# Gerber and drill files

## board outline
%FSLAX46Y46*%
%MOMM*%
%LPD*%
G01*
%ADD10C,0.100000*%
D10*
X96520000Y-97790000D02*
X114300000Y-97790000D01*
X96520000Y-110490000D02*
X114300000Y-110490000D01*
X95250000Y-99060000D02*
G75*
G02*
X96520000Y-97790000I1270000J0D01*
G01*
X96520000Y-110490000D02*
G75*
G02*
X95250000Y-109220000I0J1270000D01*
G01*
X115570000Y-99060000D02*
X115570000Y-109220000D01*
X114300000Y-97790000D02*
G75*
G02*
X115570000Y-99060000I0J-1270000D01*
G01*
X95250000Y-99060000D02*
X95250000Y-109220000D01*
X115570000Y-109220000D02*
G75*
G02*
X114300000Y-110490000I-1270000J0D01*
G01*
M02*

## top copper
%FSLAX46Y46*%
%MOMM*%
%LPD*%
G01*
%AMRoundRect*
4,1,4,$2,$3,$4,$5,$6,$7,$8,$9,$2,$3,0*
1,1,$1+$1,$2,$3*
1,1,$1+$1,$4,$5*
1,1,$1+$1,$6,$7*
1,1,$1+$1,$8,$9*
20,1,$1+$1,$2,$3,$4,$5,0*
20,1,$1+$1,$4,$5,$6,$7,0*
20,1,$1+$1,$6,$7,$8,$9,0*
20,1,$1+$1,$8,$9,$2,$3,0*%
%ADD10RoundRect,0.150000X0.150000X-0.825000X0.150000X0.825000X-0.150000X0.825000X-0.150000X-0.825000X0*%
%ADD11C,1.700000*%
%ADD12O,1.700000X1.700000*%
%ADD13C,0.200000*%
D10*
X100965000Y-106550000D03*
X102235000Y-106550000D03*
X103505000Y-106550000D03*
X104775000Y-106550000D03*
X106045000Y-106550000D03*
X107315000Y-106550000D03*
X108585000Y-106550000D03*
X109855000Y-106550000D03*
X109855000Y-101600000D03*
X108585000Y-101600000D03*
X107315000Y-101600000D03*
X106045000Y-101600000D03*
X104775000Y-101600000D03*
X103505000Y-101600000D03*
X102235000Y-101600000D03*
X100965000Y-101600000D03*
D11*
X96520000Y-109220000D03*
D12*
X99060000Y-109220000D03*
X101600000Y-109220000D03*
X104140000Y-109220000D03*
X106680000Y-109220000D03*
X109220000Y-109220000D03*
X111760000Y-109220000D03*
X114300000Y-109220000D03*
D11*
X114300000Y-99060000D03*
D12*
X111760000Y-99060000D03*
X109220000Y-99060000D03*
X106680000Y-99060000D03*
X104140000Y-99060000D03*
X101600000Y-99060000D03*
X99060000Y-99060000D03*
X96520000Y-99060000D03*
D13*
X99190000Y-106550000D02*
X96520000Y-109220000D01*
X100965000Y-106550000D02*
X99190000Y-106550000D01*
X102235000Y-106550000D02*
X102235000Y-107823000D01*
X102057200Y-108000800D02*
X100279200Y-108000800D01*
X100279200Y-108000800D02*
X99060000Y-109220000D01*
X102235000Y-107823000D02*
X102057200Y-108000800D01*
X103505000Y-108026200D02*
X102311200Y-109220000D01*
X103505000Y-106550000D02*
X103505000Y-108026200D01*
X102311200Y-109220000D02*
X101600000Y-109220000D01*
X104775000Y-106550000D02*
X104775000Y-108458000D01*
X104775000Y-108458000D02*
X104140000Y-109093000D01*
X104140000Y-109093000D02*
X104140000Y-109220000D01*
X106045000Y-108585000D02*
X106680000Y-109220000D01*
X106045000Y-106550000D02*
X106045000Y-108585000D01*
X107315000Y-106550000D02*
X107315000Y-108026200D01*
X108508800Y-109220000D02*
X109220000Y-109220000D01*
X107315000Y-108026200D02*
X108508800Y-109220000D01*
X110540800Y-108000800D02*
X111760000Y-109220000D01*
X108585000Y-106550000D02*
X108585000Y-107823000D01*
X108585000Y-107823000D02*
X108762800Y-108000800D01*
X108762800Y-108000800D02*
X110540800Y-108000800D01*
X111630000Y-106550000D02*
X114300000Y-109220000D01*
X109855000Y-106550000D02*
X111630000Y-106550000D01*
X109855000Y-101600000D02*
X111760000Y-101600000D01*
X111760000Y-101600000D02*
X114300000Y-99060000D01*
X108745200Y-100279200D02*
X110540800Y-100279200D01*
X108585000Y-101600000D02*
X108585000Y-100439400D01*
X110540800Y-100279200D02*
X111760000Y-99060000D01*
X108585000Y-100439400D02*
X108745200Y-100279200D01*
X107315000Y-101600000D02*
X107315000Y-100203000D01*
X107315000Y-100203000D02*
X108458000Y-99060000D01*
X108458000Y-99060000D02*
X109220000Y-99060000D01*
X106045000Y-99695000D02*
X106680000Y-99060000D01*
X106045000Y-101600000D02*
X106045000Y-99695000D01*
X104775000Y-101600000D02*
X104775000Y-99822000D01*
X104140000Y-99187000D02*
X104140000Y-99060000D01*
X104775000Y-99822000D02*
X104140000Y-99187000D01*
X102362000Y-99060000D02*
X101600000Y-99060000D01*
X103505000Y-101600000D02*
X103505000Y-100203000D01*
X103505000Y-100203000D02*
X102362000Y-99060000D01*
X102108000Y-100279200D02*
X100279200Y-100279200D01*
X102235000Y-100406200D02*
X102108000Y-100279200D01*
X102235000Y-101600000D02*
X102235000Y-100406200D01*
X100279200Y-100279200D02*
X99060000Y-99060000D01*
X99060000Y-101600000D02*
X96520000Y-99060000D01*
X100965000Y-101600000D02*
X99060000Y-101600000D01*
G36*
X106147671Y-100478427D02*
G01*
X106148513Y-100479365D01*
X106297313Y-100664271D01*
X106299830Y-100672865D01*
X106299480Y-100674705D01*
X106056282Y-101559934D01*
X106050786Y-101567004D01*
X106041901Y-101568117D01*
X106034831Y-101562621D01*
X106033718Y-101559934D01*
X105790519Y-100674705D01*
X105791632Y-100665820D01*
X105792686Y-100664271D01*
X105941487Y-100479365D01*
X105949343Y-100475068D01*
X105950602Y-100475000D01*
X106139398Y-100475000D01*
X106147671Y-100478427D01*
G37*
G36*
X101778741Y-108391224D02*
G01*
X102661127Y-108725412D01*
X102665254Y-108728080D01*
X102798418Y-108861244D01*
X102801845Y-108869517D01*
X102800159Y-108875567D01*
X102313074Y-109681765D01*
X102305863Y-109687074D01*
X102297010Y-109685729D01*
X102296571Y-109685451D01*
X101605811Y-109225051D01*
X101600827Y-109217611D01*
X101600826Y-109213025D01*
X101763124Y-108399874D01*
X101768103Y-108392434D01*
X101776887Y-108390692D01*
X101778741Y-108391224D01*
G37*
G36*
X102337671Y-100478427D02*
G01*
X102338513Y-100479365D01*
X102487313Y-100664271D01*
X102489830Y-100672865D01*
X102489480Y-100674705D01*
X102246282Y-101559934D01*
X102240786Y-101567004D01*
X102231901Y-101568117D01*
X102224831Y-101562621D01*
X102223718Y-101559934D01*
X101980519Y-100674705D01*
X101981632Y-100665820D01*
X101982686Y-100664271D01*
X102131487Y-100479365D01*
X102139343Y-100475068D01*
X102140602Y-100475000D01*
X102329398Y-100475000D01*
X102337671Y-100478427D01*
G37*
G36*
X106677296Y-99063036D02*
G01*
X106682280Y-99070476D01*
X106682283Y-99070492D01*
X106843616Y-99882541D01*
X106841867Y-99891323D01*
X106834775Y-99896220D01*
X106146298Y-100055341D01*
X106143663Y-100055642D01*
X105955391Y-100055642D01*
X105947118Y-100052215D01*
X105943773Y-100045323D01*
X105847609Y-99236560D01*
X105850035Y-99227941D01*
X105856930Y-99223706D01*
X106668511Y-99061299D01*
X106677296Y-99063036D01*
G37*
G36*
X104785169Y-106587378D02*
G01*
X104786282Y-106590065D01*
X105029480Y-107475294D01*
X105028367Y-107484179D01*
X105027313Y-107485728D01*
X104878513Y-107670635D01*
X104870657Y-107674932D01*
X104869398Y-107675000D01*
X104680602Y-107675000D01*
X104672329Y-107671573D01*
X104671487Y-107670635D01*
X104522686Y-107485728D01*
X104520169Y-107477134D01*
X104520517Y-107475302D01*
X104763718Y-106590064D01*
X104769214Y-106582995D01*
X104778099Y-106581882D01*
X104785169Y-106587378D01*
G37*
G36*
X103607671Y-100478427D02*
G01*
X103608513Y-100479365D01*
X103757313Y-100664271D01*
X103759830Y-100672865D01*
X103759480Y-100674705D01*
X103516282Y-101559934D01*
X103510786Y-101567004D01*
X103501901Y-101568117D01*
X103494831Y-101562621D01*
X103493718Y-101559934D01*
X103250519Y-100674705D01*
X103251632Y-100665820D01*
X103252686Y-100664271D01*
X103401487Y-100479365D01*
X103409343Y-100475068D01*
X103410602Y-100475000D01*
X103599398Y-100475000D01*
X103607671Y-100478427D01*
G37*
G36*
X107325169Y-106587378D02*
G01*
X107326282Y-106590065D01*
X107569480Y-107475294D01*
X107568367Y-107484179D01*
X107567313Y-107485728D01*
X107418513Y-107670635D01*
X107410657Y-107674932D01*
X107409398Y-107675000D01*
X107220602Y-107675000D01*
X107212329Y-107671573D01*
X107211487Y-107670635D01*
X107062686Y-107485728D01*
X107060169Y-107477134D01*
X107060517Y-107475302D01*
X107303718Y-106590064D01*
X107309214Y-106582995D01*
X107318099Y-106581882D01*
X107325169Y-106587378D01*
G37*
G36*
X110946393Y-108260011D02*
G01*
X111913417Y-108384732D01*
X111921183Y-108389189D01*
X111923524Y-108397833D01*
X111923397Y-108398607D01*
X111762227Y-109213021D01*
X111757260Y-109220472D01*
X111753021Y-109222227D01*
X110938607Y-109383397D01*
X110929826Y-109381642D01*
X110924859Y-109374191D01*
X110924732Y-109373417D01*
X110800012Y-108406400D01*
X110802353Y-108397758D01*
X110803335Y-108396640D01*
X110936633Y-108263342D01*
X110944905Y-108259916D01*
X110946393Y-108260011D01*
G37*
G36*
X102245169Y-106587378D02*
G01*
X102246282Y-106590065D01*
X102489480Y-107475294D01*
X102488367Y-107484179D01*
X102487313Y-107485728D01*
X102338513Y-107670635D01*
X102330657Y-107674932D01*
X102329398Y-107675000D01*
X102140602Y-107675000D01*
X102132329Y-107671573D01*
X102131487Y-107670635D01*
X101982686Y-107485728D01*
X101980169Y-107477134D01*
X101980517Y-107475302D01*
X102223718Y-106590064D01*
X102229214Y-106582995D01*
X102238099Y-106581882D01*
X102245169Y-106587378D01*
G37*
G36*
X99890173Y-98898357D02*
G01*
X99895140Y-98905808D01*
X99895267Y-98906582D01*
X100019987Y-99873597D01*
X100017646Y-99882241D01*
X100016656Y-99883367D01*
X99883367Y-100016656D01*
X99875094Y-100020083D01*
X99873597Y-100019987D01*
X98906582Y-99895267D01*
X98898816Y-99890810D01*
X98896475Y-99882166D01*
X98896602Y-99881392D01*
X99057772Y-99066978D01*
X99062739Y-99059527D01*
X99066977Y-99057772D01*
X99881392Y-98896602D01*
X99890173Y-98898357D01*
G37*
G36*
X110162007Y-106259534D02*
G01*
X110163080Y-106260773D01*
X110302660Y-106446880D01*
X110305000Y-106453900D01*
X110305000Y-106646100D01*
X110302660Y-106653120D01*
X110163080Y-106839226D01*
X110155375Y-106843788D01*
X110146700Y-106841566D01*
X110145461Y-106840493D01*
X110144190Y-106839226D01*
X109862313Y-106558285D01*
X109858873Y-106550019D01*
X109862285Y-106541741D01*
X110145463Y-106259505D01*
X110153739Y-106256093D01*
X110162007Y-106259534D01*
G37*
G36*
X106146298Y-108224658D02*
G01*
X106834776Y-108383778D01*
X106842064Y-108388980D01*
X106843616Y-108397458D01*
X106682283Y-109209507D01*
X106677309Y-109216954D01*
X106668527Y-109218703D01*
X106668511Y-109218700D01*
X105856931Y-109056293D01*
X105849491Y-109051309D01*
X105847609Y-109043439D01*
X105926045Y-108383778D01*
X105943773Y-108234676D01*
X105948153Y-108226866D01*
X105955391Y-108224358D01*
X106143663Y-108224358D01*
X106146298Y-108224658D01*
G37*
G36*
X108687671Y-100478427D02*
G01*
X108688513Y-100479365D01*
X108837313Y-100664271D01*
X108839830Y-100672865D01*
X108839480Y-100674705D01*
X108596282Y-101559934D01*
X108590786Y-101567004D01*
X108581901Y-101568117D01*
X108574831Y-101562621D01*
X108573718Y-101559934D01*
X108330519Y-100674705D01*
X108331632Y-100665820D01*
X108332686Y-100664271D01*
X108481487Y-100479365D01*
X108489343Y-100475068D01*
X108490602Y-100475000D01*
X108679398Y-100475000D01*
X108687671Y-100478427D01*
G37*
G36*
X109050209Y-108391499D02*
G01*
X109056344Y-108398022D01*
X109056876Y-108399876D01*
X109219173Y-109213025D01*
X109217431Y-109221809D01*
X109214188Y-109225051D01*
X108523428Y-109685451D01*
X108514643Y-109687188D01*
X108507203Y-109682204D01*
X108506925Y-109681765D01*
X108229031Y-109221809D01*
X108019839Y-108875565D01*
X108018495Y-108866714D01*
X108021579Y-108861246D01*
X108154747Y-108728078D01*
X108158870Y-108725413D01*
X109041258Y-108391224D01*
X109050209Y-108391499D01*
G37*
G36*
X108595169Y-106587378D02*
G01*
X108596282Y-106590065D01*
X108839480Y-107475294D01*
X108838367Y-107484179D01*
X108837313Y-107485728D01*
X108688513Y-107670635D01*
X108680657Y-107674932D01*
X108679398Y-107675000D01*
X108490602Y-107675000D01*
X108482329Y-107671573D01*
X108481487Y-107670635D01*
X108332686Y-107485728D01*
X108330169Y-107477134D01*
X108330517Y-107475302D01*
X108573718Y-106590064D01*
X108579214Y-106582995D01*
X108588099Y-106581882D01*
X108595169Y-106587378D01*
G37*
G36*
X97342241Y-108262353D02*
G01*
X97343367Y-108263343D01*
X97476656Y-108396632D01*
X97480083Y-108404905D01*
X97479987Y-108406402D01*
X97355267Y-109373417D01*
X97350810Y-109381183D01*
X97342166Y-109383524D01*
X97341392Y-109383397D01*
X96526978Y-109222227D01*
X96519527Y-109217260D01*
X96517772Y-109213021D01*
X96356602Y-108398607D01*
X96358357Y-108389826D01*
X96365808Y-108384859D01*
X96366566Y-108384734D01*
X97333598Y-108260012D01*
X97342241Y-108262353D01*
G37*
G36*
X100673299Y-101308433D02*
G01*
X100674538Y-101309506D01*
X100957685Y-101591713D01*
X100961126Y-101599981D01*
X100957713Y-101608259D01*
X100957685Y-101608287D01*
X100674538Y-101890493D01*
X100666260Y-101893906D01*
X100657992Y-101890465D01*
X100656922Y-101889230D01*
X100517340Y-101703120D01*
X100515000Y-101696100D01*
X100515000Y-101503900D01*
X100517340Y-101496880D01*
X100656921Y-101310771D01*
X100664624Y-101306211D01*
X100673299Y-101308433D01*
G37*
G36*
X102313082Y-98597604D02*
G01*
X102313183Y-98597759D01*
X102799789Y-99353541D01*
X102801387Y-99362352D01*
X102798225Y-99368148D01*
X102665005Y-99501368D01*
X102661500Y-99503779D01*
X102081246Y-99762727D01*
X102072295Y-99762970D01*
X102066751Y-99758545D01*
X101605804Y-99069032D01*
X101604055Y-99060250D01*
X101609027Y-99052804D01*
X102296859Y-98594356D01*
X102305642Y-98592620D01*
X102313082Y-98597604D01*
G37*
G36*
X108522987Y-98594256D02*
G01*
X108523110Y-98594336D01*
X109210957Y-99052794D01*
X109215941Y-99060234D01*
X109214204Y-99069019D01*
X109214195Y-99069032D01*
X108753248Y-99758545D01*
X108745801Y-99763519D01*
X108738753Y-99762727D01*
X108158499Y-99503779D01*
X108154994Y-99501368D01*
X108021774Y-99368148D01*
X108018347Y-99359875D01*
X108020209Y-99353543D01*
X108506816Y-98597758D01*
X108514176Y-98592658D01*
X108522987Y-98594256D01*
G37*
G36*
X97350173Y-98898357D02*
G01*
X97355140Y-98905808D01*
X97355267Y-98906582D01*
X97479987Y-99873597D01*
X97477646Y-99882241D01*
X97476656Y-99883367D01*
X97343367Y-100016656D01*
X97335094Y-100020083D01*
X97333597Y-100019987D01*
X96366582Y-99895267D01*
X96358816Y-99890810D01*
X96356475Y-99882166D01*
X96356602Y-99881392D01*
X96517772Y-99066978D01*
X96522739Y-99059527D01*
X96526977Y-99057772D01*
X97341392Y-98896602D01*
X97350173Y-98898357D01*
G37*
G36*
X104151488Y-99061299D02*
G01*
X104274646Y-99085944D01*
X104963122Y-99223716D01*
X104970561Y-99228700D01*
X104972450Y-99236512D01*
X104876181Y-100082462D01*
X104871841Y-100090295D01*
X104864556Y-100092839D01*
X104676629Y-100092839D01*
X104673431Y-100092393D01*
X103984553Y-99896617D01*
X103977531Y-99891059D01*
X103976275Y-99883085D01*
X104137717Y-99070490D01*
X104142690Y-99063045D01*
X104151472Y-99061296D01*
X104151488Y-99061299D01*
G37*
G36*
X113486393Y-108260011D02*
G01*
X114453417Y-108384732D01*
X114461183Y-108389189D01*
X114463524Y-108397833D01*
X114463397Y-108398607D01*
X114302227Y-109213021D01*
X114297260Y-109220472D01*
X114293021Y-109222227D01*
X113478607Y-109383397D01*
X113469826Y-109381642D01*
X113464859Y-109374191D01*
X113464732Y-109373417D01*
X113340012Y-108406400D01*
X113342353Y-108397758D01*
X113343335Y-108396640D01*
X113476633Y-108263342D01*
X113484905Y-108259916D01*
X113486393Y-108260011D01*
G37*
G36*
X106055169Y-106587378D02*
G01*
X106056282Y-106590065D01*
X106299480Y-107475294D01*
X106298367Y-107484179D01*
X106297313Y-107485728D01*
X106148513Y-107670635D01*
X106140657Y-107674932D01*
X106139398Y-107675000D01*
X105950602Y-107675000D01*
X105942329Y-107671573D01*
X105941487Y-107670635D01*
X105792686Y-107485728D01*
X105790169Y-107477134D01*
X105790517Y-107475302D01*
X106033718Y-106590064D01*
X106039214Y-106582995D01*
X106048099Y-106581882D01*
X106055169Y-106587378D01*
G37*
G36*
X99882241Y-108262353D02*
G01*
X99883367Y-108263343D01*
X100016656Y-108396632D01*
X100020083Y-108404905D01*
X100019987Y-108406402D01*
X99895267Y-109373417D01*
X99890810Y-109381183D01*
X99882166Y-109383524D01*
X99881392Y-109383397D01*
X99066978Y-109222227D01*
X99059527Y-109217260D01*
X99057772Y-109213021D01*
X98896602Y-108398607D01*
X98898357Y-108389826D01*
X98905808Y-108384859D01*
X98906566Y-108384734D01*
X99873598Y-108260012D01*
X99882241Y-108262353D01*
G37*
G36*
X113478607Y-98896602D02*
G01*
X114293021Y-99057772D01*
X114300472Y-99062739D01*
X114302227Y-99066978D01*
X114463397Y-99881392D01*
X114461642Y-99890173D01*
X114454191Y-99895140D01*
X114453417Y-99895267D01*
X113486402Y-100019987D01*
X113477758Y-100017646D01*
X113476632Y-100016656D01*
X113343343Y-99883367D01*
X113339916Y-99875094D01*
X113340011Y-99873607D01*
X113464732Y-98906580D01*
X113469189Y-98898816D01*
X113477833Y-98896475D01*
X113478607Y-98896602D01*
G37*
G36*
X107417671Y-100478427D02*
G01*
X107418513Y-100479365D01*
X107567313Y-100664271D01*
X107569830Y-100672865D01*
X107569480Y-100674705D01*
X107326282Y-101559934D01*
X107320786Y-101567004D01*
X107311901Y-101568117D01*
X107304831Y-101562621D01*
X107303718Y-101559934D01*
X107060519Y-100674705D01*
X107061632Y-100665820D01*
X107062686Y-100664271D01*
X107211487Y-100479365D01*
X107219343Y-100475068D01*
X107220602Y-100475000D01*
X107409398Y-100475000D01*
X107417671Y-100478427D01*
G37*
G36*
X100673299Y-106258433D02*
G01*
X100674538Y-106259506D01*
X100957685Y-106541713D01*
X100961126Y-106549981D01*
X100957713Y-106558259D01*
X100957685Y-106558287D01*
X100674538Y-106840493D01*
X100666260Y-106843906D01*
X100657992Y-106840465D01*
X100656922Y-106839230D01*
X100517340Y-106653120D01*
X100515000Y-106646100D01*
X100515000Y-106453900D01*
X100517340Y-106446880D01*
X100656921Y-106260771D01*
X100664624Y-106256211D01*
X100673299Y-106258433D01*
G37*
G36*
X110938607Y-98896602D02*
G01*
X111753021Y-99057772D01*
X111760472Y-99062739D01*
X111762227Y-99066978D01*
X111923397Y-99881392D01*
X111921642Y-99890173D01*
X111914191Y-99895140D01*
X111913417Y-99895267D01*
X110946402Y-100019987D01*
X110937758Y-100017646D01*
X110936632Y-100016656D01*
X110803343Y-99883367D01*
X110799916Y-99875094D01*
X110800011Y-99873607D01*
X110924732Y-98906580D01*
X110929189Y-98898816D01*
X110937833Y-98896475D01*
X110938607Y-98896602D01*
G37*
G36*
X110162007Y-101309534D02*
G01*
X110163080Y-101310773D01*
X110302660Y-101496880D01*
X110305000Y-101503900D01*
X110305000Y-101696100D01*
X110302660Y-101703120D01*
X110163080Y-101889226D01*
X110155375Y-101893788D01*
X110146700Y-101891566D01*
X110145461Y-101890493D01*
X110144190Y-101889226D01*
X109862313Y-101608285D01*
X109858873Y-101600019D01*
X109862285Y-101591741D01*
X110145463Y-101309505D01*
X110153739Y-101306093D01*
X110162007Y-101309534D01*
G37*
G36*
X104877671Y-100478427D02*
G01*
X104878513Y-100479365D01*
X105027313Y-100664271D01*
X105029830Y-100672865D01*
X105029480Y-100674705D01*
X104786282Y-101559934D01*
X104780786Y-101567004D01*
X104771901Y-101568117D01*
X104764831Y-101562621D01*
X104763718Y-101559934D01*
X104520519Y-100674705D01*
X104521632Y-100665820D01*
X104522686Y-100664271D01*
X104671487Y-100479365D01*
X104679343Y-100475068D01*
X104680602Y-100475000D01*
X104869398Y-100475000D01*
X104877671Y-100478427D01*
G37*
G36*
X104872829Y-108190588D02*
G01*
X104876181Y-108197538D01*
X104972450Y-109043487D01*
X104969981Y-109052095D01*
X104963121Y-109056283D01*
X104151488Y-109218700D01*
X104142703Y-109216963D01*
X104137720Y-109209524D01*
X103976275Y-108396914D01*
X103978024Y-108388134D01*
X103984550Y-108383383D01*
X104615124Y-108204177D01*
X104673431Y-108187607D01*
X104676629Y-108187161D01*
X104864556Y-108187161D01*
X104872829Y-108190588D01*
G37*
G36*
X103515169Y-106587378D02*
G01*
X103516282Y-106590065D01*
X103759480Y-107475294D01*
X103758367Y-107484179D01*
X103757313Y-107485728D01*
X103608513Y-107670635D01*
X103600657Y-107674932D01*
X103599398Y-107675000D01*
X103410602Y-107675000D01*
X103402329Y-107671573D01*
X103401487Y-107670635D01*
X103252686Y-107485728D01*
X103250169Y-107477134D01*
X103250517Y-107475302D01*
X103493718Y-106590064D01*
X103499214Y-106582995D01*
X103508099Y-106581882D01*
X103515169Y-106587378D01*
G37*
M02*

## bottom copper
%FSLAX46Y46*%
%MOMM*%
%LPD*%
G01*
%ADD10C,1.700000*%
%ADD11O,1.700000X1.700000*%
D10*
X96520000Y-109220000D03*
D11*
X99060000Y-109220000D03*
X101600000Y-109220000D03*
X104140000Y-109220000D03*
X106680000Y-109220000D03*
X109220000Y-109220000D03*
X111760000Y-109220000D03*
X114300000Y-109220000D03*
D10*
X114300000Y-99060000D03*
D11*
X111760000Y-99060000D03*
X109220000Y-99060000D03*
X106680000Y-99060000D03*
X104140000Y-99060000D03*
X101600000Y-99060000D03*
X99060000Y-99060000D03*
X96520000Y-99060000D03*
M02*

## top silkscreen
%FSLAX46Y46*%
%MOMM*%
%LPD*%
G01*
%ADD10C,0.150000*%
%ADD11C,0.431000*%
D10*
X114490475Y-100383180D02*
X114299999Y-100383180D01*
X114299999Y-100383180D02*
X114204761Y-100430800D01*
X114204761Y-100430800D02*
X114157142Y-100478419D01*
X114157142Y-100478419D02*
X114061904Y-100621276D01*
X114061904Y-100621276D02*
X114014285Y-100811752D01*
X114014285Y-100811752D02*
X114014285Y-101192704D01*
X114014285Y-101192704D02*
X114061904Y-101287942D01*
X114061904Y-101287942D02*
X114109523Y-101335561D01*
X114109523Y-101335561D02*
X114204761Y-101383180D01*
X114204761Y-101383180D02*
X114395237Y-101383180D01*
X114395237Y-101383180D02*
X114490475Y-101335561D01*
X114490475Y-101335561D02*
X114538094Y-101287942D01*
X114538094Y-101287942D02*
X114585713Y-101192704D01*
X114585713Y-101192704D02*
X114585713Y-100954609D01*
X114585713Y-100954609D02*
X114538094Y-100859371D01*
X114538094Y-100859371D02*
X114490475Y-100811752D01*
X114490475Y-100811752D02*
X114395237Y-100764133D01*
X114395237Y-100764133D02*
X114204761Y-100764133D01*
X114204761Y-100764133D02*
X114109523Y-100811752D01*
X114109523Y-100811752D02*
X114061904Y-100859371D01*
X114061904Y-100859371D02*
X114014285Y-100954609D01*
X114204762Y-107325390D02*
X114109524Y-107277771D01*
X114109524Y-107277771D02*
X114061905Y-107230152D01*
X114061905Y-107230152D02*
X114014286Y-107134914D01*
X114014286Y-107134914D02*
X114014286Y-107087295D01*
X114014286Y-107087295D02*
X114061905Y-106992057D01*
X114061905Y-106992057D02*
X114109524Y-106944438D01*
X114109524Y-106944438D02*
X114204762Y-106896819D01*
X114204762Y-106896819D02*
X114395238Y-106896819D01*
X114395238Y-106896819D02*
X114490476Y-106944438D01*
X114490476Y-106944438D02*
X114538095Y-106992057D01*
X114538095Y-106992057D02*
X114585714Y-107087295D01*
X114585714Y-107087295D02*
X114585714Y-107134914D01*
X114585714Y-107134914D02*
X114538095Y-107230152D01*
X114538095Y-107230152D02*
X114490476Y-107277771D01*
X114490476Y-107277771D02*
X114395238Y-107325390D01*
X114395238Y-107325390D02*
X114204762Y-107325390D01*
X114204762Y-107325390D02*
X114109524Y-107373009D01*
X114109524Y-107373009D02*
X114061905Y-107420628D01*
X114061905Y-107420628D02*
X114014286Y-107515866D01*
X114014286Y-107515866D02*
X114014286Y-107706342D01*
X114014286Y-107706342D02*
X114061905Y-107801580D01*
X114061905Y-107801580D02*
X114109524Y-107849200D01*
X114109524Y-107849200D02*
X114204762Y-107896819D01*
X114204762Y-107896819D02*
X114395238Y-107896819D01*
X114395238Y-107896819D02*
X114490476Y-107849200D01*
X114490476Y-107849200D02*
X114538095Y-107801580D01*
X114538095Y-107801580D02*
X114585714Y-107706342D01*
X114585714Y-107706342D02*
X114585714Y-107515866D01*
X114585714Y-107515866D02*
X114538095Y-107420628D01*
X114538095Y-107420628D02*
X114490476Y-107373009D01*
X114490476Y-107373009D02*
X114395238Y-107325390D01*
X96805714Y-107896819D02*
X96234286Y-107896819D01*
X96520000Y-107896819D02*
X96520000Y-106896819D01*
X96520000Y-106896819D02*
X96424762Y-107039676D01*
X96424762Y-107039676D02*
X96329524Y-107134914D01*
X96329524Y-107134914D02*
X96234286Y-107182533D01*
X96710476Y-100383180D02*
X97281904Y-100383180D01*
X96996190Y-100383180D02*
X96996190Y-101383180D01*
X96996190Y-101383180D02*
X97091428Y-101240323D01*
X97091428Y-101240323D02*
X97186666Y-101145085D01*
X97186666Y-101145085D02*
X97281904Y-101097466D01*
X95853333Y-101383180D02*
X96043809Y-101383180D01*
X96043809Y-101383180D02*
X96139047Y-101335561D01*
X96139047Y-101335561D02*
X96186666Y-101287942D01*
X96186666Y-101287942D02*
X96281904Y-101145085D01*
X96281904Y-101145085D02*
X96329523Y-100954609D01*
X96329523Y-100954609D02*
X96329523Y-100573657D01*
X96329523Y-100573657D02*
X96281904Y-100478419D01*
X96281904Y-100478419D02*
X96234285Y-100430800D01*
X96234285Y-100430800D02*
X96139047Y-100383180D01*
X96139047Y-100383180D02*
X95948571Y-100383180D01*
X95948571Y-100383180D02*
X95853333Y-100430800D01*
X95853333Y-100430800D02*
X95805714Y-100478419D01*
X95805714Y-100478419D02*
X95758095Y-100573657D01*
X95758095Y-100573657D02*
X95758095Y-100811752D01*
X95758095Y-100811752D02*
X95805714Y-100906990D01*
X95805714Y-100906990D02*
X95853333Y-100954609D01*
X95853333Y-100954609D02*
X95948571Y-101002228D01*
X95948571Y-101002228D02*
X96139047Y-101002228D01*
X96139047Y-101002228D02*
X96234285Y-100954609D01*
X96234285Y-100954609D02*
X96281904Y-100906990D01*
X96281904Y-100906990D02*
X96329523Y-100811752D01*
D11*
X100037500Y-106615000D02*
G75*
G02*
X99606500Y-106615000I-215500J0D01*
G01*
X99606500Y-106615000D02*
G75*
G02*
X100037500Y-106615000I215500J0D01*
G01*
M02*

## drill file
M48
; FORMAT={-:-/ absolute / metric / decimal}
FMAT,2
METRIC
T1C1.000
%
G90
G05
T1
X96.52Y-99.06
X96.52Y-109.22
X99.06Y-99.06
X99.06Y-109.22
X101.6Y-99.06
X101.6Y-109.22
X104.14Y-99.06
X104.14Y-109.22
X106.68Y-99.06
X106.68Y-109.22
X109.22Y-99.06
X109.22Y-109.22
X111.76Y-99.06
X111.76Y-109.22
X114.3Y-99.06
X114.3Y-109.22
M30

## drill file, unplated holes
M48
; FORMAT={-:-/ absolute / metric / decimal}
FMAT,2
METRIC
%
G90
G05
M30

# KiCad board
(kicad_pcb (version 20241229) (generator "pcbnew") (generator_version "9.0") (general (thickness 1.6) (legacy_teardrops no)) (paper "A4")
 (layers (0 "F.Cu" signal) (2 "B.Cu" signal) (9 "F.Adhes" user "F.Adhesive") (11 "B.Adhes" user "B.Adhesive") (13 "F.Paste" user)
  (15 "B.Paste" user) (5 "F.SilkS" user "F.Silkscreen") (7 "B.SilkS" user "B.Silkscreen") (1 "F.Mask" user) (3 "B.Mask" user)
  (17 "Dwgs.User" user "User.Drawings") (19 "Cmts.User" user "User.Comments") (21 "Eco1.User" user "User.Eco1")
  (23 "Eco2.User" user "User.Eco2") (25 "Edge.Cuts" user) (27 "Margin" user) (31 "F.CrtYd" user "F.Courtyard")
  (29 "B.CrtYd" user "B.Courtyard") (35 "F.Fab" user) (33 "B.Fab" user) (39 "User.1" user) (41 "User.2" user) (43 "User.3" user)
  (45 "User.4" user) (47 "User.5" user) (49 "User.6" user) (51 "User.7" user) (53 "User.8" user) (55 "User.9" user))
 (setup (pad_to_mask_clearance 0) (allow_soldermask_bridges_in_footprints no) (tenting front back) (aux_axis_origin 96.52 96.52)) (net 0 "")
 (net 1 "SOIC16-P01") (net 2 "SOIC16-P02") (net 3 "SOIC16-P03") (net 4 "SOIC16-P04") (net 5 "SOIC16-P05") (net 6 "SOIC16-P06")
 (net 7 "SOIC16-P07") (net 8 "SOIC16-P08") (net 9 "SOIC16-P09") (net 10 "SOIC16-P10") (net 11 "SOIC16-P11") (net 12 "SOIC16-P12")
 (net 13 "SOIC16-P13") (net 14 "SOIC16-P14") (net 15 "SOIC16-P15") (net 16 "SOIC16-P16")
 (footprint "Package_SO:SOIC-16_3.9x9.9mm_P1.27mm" (layer "F.Cu") (at 105.41 104.075 90)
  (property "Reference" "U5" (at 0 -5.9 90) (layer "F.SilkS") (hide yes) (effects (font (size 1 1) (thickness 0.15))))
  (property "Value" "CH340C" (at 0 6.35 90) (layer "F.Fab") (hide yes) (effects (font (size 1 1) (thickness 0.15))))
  (fp_circle (center -2.54 -5.588) (end -2.159 -5.588) (stroke (width 0.1) (type solid)) (fill yes) (layer "F.SilkS"))
  (pad "1" smd roundrect (at -2.475 -4.445 90) (size 1.95 0.6) (layers "F.Cu" "F.Mask" "F.Paste") (roundrect_rratio 0.25)
   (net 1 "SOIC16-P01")
   (teardrops (best_length_ratio 0.25) (max_length 1) (best_width_ratio 1) (max_width 2) (curved_edges no) (filter_ratio 0.9) (enabled yes)
    (allow_two_segments yes) (prefer_zone_connections yes)))
  (pad "2" smd roundrect (at -2.475 -3.175 90) (size 1.95 0.6) (layers "F.Cu" "F.Mask" "F.Paste") (roundrect_rratio 0.25)
   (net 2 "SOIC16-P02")
   (teardrops (best_length_ratio 0.25) (max_length 1) (best_width_ratio 1) (max_width 2) (curved_edges no) (filter_ratio 0.9) (enabled yes)
    (allow_two_segments yes) (prefer_zone_connections yes)))
  (pad "3" smd roundrect (at -2.475 -1.905 90) (size 1.95 0.6) (layers "F.Cu" "F.Mask" "F.Paste") (roundrect_rratio 0.25)
   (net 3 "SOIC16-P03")
   (teardrops (best_length_ratio 0.25) (max_length 1) (best_width_ratio 1) (max_width 2) (curved_edges no) (filter_ratio 0.9) (enabled yes)
    (allow_two_segments yes) (prefer_zone_connections yes)))
  (pad "4" smd roundrect (at -2.475 -0.635 90) (size 1.95 0.6) (layers "F.Cu" "F.Mask" "F.Paste") (roundrect_rratio 0.25)
   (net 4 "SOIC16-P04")
   (teardrops (best_length_ratio 0.25) (max_length 1) (best_width_ratio 1) (max_width 2) (curved_edges no) (filter_ratio 0.9) (enabled yes)
    (allow_two_segments yes) (prefer_zone_connections yes)))
  (pad "5" smd roundrect (at -2.475 0.635 90) (size 1.95 0.6) (layers "F.Cu" "F.Mask" "F.Paste") (roundrect_rratio 0.25)
   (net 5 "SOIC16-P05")
   (teardrops (best_length_ratio 0.25) (max_length 1) (best_width_ratio 1) (max_width 2) (curved_edges no) (filter_ratio 0.9) (enabled yes)
    (allow_two_segments yes) (prefer_zone_connections yes)))
  (pad "6" smd roundrect (at -2.475 1.905 90) (size 1.95 0.6) (layers "F.Cu" "F.Mask" "F.Paste") (roundrect_rratio 0.25)
   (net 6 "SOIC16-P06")
   (teardrops (best_length_ratio 0.25) (max_length 1) (best_width_ratio 1) (max_width 2) (curved_edges no) (filter_ratio 0.9) (enabled yes)
    (allow_two_segments yes) (prefer_zone_connections yes)))
  (pad "7" smd roundrect (at -2.475 3.175 90) (size 1.95 0.6) (layers "F.Cu" "F.Mask" "F.Paste") (roundrect_rratio 0.25)
   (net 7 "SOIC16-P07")
   (teardrops (best_length_ratio 0.25) (max_length 1) (best_width_ratio 1) (max_width 2) (curved_edges no) (filter_ratio 0.9) (enabled yes)
    (allow_two_segments yes) (prefer_zone_connections yes)))
  (pad "8" smd roundrect (at -2.475 4.445 90) (size 1.95 0.6) (layers "F.Cu" "F.Mask" "F.Paste") (roundrect_rratio 0.25)
   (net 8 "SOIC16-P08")
   (teardrops (best_length_ratio 0.25) (max_length 1) (best_width_ratio 1) (max_width 2) (curved_edges no) (filter_ratio 0.9) (enabled yes)
    (allow_two_segments yes) (prefer_zone_connections yes)))
  (pad "9" smd roundrect (at 2.475 4.445 90) (size 1.95 0.6) (layers "F.Cu" "F.Mask" "F.Paste") (roundrect_rratio 0.25) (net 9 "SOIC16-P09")
   (teardrops (best_length_ratio 0.25) (max_length 1) (best_width_ratio 1) (max_width 2) (curved_edges no) (filter_ratio 0.9) (enabled yes)
    (allow_two_segments yes) (prefer_zone_connections yes)))
  (pad "10" smd roundrect (at 2.475 3.175 90) (size 1.95 0.6) (layers "F.Cu" "F.Mask" "F.Paste") (roundrect_rratio 0.25)
   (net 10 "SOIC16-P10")
   (teardrops (best_length_ratio 0.25) (max_length 1) (best_width_ratio 1) (max_width 2) (curved_edges no) (filter_ratio 0.9) (enabled yes)
    (allow_two_segments yes) (prefer_zone_connections yes)))
  (pad "11" smd roundrect (at 2.475 1.905 90) (size 1.95 0.6) (layers "F.Cu" "F.Mask" "F.Paste") (roundrect_rratio 0.25)
   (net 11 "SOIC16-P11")
   (teardrops (best_length_ratio 0.25) (max_length 1) (best_width_ratio 1) (max_width 2) (curved_edges no) (filter_ratio 0.9) (enabled yes)
    (allow_two_segments yes) (prefer_zone_connections yes)))
  (pad "12" smd roundrect (at 2.475 0.635 90) (size 1.95 0.6) (layers "F.Cu" "F.Mask" "F.Paste") (roundrect_rratio 0.25)
   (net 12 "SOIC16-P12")
   (teardrops (best_length_ratio 0.25) (max_length 1) (best_width_ratio 1) (max_width 2) (curved_edges no) (filter_ratio 0.9) (enabled yes)
    (allow_two_segments yes) (prefer_zone_connections yes)))
  (pad "13" smd roundrect (at 2.475 -0.635 90) (size 1.95 0.6) (layers "F.Cu" "F.Mask" "F.Paste") (roundrect_rratio 0.25)
   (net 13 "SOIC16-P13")
   (teardrops (best_length_ratio 0.25) (max_length 1) (best_width_ratio 1) (max_width 2) (curved_edges no) (filter_ratio 0.9) (enabled yes)
    (allow_two_segments yes) (prefer_zone_connections yes)))
  (pad "14" smd roundrect (at 2.475 -1.905 90) (size 1.95 0.6) (layers "F.Cu" "F.Mask" "F.Paste") (roundrect_rratio 0.25)
   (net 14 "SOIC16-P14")
   (teardrops (best_length_ratio 0.25) (max_length 1) (best_width_ratio 1) (max_width 2) (curved_edges no) (filter_ratio 0.9) (enabled yes)
    (allow_two_segments yes) (prefer_zone_connections yes)))
  (pad "15" smd roundrect (at 2.475 -3.175 90) (size 1.95 0.6) (layers "F.Cu" "F.Mask" "F.Paste") (roundrect_rratio 0.25)
   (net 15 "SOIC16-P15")
   (teardrops (best_length_ratio 0.25) (max_length 1) (best_width_ratio 1) (max_width 2) (curved_edges no) (filter_ratio 0.9) (enabled yes)
    (allow_two_segments yes) (prefer_zone_connections yes)))
  (pad "16" smd roundrect (at 2.475 -4.445 90) (size 1.95 0.6) (layers "F.Cu" "F.Mask" "F.Paste") (roundrect_rratio 0.25)
   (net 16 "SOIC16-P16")
   (teardrops (best_length_ratio 0.25) (max_length 1) (best_width_ratio 1) (max_width 2) (curved_edges no) (filter_ratio 0.9) (enabled yes)
    (allow_two_segments yes) (prefer_zone_connections yes))))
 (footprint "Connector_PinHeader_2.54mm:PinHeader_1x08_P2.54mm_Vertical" (layer "B.Cu") (at 96.52 109.22 -90)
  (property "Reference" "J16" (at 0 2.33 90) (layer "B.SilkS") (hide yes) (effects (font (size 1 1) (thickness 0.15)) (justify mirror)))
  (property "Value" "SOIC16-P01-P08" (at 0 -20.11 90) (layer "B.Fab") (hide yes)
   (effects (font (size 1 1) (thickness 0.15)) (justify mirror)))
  (pad "1" thru_hole circle (at 0 0 270) (size 1.7 1.7) (drill 1) (layers "*.Cu" "*.Mask") (remove_unused_layers no) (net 1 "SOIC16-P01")
   (teardrops (best_length_ratio 0.25) (max_length 1) (best_width_ratio 1) (max_width 2) (curved_edges no) (filter_ratio 0.9) (enabled yes)
    (allow_two_segments yes) (prefer_zone_connections yes)))
  (pad "2" thru_hole oval (at 0 -2.54 270) (size 1.7 1.7) (drill 1) (layers "*.Cu" "*.Mask") (remove_unused_layers no) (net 2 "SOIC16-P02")
   (teardrops (best_length_ratio 0.25) (max_length 1) (best_width_ratio 1) (max_width 2) (curved_edges no) (filter_ratio 0.9) (enabled yes)
    (allow_two_segments yes) (prefer_zone_connections yes)))
  (pad "3" thru_hole oval (at 0 -5.08 270) (size 1.7 1.7) (drill 1) (layers "*.Cu" "*.Mask") (remove_unused_layers no) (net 3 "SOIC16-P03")
   (teardrops (best_length_ratio 0.25) (max_length 1) (best_width_ratio 1) (max_width 2) (curved_edges no) (filter_ratio 0.9) (enabled yes)
    (allow_two_segments yes) (prefer_zone_connections yes)))
  (pad "4" thru_hole oval (at 0 -7.62 270) (size 1.7 1.7) (drill 1) (layers "*.Cu" "*.Mask") (remove_unused_layers no) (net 4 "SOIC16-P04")
   (teardrops (best_length_ratio 0.25) (max_length 1) (best_width_ratio 1) (max_width 2) (curved_edges no) (filter_ratio 0.9) (enabled yes)
    (allow_two_segments yes) (prefer_zone_connections yes)))
  (pad "5" thru_hole oval (at 0 -10.16 270) (size 1.7 1.7) (drill 1) (layers "*.Cu" "*.Mask") (remove_unused_layers no) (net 5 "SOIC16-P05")
   (teardrops (best_length_ratio 0.25) (max_length 1) (best_width_ratio 1) (max_width 2) (curved_edges no) (filter_ratio 0.9) (enabled yes)
    (allow_two_segments yes) (prefer_zone_connections yes)))
  (pad "6" thru_hole oval (at 0 -12.7 270) (size 1.7 1.7) (drill 1) (layers "*.Cu" "*.Mask") (remove_unused_layers no) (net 6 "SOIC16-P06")
   (teardrops (best_length_ratio 0.25) (max_length 1) (best_width_ratio 1) (max_width 2) (curved_edges no) (filter_ratio 0.9) (enabled yes)
    (allow_two_segments yes) (prefer_zone_connections yes)))
  (pad "7" thru_hole oval (at 0 -15.24 270) (size 1.7 1.7) (drill 1) (layers "*.Cu" "*.Mask") (remove_unused_layers no) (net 7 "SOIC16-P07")
   (teardrops (best_length_ratio 0.25) (max_length 1) (best_width_ratio 1) (max_width 2) (curved_edges no) (filter_ratio 0.9) (enabled yes)
    (allow_two_segments yes) (prefer_zone_connections yes)))
  (pad "8" thru_hole oval (at 0 -17.78 270) (size 1.7 1.7) (drill 1) (layers "*.Cu" "*.Mask") (remove_unused_layers no) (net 8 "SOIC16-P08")
   (teardrops (best_length_ratio 0.25) (max_length 1) (best_width_ratio 1) (max_width 2) (curved_edges no) (filter_ratio 0.9) (enabled yes)
    (allow_two_segments yes) (prefer_zone_connections yes))))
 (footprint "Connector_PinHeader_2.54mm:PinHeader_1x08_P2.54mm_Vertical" (layer "B.Cu") (at 114.3 99.06 90)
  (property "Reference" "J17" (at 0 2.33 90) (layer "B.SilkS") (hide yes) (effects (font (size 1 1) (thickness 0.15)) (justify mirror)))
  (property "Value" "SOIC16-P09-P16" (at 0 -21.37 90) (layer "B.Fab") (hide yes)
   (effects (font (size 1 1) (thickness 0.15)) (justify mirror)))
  (pad "1" thru_hole circle (at 0 0 90) (size 1.7 1.7) (drill 1) (layers "*.Cu" "*.Mask") (remove_unused_layers no) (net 9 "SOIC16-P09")
   (teardrops (best_length_ratio 0.25) (max_length 1) (best_width_ratio 1) (max_width 2) (curved_edges no) (filter_ratio 0.9) (enabled yes)
    (allow_two_segments yes) (prefer_zone_connections yes)))
  (pad "2" thru_hole oval (at 0 -2.54 90) (size 1.7 1.7) (drill 1) (layers "*.Cu" "*.Mask") (remove_unused_layers no) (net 10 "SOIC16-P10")
   (teardrops (best_length_ratio 0.25) (max_length 1) (best_width_ratio 1) (max_width 2) (curved_edges no) (filter_ratio 0.9) (enabled yes)
    (allow_two_segments yes) (prefer_zone_connections yes)))
  (pad "3" thru_hole oval (at 0 -5.08 90) (size 1.7 1.7) (drill 1) (layers "*.Cu" "*.Mask") (remove_unused_layers no) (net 11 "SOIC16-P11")
   (teardrops (best_length_ratio 0.25) (max_length 1) (best_width_ratio 1) (max_width 2) (curved_edges no) (filter_ratio 0.9) (enabled yes)
    (allow_two_segments yes) (prefer_zone_connections yes)))
  (pad "4" thru_hole oval (at 0 -7.62 90) (size 1.7 1.7) (drill 1) (layers "*.Cu" "*.Mask") (remove_unused_layers no) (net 12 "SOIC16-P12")
   (teardrops (best_length_ratio 0.25) (max_length 1) (best_width_ratio 1) (max_width 2) (curved_edges no) (filter_ratio 0.9) (enabled yes)
    (allow_two_segments yes) (prefer_zone_connections yes)))
  (pad "5" thru_hole oval (at 0 -10.16 90) (size 1.7 1.7) (drill 1) (layers "*.Cu" "*.Mask") (remove_unused_layers no) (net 13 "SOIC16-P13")
   (teardrops (best_length_ratio 0.25) (max_length 1) (best_width_ratio 1) (max_width 2) (curved_edges no) (filter_ratio 0.9) (enabled yes)
    (allow_two_segments yes) (prefer_zone_connections yes)))
  (pad "6" thru_hole oval (at 0 -12.7 90) (size 1.7 1.7) (drill 1) (layers "*.Cu" "*.Mask") (remove_unused_layers no) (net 14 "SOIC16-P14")
   (teardrops (best_length_ratio 0.25) (max_length 1) (best_width_ratio 1) (max_width 2) (curved_edges no) (filter_ratio 0.9) (enabled yes)
    (allow_two_segments yes) (prefer_zone_connections yes)))
  (pad "7" thru_hole oval (at 0 -15.24 90) (size 1.7 1.7) (drill 1) (layers "*.Cu" "*.Mask") (remove_unused_layers no) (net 15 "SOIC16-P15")
   (teardrops (best_length_ratio 0.25) (max_length 1) (best_width_ratio 1) (max_width 2) (curved_edges no) (filter_ratio 0.9) (enabled yes)
    (allow_two_segments yes) (prefer_zone_connections yes)))
  (pad "8" thru_hole oval (at 0 -17.78 90) (size 1.7 1.7) (drill 1) (layers "*.Cu" "*.Mask") (remove_unused_layers no) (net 16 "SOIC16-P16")
   (teardrops (best_length_ratio 0.25) (max_length 1) (best_width_ratio 1) (max_width 2) (curved_edges no) (filter_ratio 0.9) (enabled yes)
    (allow_two_segments yes) (prefer_zone_connections yes))))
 (gr_line (start 96.52 97.79) (end 114.3 97.79) (stroke (width 0.1) (type solid)) (layer "Edge.Cuts"))
 (gr_line (start 96.52 110.49) (end 114.3 110.49) (stroke (width 0.1) (type solid)) (layer "Edge.Cuts"))
 (gr_arc (start 95.25 99.06) (mid 95.621974 98.161974) (end 96.52 97.79) (stroke (width 0.1) (type default)) (layer "Edge.Cuts"))
 (gr_arc (start 96.52 110.49) (mid 95.621974 110.118026) (end 95.25 109.22) (stroke (width 0.1) (type default)) (layer "Edge.Cuts"))
 (gr_line (start 115.57 99.06) (end 115.57 109.22) (stroke (width 0.1) (type solid)) (layer "Edge.Cuts"))
 (gr_arc (start 114.3 97.79) (mid 115.198026 98.161974) (end 115.57 99.06) (stroke (width 0.1) (type default)) (layer "Edge.Cuts"))
 (gr_line (start 95.25 99.06) (end 95.25 109.22) (stroke (width 0.1) (type solid)) (layer "Edge.Cuts"))
 (gr_arc (start 115.57 109.22) (mid 115.198026 110.118026) (end 114.3 110.49) (stroke (width 0.1) (type default)) (layer "Edge.Cuts"))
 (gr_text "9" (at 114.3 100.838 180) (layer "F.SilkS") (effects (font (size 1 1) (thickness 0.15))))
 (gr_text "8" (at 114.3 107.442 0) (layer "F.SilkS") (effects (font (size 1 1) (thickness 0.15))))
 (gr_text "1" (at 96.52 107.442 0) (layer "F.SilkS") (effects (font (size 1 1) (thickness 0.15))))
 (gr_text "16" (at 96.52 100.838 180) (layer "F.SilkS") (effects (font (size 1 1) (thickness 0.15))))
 (segment (start 99.19 106.55) (end 96.52 109.22) (width 0.2) (layer "F.Cu") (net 1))
 (segment (start 100.965 106.55) (end 99.19 106.55) (width 0.2) (layer "F.Cu") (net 1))
 (segment (start 102.235 106.55) (end 102.235 107.823) (width 0.2) (layer "F.Cu") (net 2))
 (segment (start 102.0572 108.0008) (end 100.2792 108.0008) (width 0.2) (layer "F.Cu") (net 2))
 (segment (start 100.2792 108.0008) (end 99.06 109.22) (width 0.2) (layer "F.Cu") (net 2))
 (segment (start 102.235 107.823) (end 102.0572 108.0008) (width 0.2) (layer "F.Cu") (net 2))
 (segment (start 103.505 108.0262) (end 102.3112 109.22) (width 0.2) (layer "F.Cu") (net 3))
 (segment (start 103.505 106.55) (end 103.505 108.0262) (width 0.2) (layer "F.Cu") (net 3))
 (segment (start 102.3112 109.22) (end 101.6 109.22) (width 0.2) (layer "F.Cu") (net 3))
 (segment (start 104.775 106.55) (end 104.775 108.458) (width 0.2) (layer "F.Cu") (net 4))
 (segment (start 104.775 108.458) (end 104.14 109.093) (width 0.2) (layer "F.Cu") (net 4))
 (segment (start 104.14 109.093) (end 104.14 109.22) (width 0.2) (layer "F.Cu") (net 4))
 (segment (start 106.045 108.585) (end 106.68 109.22) (width 0.2) (layer "F.Cu") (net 5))
 (segment (start 106.045 106.55) (end 106.045 108.585) (width 0.2) (layer "F.Cu") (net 5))
 (segment (start 107.315 106.55) (end 107.315 108.0262) (width 0.2) (layer "F.Cu") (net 6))
 (segment (start 108.5088 109.22) (end 109.22 109.22) (width 0.2) (layer "F.Cu") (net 6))
 (segment (start 107.315 108.0262) (end 108.5088 109.22) (width 0.2) (layer "F.Cu") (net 6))
 (segment (start 110.5408 108.0008) (end 111.76 109.22) (width 0.2) (layer "F.Cu") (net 7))
 (segment (start 108.585 106.55) (end 108.585 107.823) (width 0.2) (layer "F.Cu") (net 7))
 (segment (start 108.585 107.823) (end 108.7628 108.0008) (width 0.2) (layer "F.Cu") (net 7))
 (segment (start 108.7628 108.0008) (end 110.5408 108.0008) (width 0.2) (layer "F.Cu") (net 7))
 (segment (start 111.63 106.55) (end 114.3 109.22) (width 0.2) (layer "F.Cu") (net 8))
 (segment (start 109.855 106.55) (end 111.63 106.55) (width 0.2) (layer "F.Cu") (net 8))
 (segment (start 109.855 101.6) (end 111.76 101.6) (width 0.2) (layer "F.Cu") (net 9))
 (segment (start 111.76 101.6) (end 114.3 99.06) (width 0.2) (layer "F.Cu") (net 9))
 (segment (start 108.7452 100.2792) (end 110.5408 100.2792) (width 0.2) (layer "F.Cu") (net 10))
 (segment (start 108.585 101.6) (end 108.585 100.4394) (width 0.2) (layer "F.Cu") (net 10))
 (segment (start 110.5408 100.2792) (end 111.76 99.06) (width 0.2) (layer "F.Cu") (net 10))
 (segment (start 108.585 100.4394) (end 108.7452 100.2792) (width 0.2) (layer "F.Cu") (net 10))
 (segment (start 107.315 101.6) (end 107.315 100.203) (width 0.2) (layer "F.Cu") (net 11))
 (segment (start 107.315 100.203) (end 108.458 99.06) (width 0.2) (layer "F.Cu") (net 11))
 (segment (start 108.458 99.06) (end 109.22 99.06) (width 0.2) (layer "F.Cu") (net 11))
 (segment (start 106.045 99.695) (end 106.68 99.06) (width 0.2) (layer "F.Cu") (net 12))
 (segment (start 106.045 101.6) (end 106.045 99.695) (width 0.2) (layer "F.Cu") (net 12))
 (segment (start 104.775 101.6) (end 104.775 99.822) (width 0.2) (layer "F.Cu") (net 13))
 (segment (start 104.14 99.187) (end 104.14 99.06) (width 0.2) (layer "F.Cu") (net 13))
 (segment (start 104.775 99.822) (end 104.14 99.187) (width 0.2) (layer "F.Cu") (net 13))
 (segment (start 102.362 99.06) (end 101.6 99.06) (width 0.2) (layer "F.Cu") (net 14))
 (segment (start 103.505 101.6) (end 103.505 100.203) (width 0.2) (layer "F.Cu") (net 14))
 (segment (start 103.505 100.203) (end 102.362 99.06) (width 0.2) (layer "F.Cu") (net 14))
 (segment (start 102.108 100.2792) (end 100.2792 100.2792) (width 0.2) (layer "F.Cu") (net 15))
 (segment (start 102.235 100.4062) (end 102.108 100.2792) (width 0.2) (layer "F.Cu") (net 15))
 (segment (start 102.235 101.6) (end 102.235 100.4062) (width 0.2) (layer "F.Cu") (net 15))
 (segment (start 100.2792 100.2792) (end 99.06 99.06) (width 0.2) (layer "F.Cu") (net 15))
 (segment (start 99.06 101.6) (end 96.52 99.06) (width 0.2) (layer "F.Cu") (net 16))
 (segment (start 100.965 101.6) (end 99.06 101.6) (width 0.2) (layer "F.Cu") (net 16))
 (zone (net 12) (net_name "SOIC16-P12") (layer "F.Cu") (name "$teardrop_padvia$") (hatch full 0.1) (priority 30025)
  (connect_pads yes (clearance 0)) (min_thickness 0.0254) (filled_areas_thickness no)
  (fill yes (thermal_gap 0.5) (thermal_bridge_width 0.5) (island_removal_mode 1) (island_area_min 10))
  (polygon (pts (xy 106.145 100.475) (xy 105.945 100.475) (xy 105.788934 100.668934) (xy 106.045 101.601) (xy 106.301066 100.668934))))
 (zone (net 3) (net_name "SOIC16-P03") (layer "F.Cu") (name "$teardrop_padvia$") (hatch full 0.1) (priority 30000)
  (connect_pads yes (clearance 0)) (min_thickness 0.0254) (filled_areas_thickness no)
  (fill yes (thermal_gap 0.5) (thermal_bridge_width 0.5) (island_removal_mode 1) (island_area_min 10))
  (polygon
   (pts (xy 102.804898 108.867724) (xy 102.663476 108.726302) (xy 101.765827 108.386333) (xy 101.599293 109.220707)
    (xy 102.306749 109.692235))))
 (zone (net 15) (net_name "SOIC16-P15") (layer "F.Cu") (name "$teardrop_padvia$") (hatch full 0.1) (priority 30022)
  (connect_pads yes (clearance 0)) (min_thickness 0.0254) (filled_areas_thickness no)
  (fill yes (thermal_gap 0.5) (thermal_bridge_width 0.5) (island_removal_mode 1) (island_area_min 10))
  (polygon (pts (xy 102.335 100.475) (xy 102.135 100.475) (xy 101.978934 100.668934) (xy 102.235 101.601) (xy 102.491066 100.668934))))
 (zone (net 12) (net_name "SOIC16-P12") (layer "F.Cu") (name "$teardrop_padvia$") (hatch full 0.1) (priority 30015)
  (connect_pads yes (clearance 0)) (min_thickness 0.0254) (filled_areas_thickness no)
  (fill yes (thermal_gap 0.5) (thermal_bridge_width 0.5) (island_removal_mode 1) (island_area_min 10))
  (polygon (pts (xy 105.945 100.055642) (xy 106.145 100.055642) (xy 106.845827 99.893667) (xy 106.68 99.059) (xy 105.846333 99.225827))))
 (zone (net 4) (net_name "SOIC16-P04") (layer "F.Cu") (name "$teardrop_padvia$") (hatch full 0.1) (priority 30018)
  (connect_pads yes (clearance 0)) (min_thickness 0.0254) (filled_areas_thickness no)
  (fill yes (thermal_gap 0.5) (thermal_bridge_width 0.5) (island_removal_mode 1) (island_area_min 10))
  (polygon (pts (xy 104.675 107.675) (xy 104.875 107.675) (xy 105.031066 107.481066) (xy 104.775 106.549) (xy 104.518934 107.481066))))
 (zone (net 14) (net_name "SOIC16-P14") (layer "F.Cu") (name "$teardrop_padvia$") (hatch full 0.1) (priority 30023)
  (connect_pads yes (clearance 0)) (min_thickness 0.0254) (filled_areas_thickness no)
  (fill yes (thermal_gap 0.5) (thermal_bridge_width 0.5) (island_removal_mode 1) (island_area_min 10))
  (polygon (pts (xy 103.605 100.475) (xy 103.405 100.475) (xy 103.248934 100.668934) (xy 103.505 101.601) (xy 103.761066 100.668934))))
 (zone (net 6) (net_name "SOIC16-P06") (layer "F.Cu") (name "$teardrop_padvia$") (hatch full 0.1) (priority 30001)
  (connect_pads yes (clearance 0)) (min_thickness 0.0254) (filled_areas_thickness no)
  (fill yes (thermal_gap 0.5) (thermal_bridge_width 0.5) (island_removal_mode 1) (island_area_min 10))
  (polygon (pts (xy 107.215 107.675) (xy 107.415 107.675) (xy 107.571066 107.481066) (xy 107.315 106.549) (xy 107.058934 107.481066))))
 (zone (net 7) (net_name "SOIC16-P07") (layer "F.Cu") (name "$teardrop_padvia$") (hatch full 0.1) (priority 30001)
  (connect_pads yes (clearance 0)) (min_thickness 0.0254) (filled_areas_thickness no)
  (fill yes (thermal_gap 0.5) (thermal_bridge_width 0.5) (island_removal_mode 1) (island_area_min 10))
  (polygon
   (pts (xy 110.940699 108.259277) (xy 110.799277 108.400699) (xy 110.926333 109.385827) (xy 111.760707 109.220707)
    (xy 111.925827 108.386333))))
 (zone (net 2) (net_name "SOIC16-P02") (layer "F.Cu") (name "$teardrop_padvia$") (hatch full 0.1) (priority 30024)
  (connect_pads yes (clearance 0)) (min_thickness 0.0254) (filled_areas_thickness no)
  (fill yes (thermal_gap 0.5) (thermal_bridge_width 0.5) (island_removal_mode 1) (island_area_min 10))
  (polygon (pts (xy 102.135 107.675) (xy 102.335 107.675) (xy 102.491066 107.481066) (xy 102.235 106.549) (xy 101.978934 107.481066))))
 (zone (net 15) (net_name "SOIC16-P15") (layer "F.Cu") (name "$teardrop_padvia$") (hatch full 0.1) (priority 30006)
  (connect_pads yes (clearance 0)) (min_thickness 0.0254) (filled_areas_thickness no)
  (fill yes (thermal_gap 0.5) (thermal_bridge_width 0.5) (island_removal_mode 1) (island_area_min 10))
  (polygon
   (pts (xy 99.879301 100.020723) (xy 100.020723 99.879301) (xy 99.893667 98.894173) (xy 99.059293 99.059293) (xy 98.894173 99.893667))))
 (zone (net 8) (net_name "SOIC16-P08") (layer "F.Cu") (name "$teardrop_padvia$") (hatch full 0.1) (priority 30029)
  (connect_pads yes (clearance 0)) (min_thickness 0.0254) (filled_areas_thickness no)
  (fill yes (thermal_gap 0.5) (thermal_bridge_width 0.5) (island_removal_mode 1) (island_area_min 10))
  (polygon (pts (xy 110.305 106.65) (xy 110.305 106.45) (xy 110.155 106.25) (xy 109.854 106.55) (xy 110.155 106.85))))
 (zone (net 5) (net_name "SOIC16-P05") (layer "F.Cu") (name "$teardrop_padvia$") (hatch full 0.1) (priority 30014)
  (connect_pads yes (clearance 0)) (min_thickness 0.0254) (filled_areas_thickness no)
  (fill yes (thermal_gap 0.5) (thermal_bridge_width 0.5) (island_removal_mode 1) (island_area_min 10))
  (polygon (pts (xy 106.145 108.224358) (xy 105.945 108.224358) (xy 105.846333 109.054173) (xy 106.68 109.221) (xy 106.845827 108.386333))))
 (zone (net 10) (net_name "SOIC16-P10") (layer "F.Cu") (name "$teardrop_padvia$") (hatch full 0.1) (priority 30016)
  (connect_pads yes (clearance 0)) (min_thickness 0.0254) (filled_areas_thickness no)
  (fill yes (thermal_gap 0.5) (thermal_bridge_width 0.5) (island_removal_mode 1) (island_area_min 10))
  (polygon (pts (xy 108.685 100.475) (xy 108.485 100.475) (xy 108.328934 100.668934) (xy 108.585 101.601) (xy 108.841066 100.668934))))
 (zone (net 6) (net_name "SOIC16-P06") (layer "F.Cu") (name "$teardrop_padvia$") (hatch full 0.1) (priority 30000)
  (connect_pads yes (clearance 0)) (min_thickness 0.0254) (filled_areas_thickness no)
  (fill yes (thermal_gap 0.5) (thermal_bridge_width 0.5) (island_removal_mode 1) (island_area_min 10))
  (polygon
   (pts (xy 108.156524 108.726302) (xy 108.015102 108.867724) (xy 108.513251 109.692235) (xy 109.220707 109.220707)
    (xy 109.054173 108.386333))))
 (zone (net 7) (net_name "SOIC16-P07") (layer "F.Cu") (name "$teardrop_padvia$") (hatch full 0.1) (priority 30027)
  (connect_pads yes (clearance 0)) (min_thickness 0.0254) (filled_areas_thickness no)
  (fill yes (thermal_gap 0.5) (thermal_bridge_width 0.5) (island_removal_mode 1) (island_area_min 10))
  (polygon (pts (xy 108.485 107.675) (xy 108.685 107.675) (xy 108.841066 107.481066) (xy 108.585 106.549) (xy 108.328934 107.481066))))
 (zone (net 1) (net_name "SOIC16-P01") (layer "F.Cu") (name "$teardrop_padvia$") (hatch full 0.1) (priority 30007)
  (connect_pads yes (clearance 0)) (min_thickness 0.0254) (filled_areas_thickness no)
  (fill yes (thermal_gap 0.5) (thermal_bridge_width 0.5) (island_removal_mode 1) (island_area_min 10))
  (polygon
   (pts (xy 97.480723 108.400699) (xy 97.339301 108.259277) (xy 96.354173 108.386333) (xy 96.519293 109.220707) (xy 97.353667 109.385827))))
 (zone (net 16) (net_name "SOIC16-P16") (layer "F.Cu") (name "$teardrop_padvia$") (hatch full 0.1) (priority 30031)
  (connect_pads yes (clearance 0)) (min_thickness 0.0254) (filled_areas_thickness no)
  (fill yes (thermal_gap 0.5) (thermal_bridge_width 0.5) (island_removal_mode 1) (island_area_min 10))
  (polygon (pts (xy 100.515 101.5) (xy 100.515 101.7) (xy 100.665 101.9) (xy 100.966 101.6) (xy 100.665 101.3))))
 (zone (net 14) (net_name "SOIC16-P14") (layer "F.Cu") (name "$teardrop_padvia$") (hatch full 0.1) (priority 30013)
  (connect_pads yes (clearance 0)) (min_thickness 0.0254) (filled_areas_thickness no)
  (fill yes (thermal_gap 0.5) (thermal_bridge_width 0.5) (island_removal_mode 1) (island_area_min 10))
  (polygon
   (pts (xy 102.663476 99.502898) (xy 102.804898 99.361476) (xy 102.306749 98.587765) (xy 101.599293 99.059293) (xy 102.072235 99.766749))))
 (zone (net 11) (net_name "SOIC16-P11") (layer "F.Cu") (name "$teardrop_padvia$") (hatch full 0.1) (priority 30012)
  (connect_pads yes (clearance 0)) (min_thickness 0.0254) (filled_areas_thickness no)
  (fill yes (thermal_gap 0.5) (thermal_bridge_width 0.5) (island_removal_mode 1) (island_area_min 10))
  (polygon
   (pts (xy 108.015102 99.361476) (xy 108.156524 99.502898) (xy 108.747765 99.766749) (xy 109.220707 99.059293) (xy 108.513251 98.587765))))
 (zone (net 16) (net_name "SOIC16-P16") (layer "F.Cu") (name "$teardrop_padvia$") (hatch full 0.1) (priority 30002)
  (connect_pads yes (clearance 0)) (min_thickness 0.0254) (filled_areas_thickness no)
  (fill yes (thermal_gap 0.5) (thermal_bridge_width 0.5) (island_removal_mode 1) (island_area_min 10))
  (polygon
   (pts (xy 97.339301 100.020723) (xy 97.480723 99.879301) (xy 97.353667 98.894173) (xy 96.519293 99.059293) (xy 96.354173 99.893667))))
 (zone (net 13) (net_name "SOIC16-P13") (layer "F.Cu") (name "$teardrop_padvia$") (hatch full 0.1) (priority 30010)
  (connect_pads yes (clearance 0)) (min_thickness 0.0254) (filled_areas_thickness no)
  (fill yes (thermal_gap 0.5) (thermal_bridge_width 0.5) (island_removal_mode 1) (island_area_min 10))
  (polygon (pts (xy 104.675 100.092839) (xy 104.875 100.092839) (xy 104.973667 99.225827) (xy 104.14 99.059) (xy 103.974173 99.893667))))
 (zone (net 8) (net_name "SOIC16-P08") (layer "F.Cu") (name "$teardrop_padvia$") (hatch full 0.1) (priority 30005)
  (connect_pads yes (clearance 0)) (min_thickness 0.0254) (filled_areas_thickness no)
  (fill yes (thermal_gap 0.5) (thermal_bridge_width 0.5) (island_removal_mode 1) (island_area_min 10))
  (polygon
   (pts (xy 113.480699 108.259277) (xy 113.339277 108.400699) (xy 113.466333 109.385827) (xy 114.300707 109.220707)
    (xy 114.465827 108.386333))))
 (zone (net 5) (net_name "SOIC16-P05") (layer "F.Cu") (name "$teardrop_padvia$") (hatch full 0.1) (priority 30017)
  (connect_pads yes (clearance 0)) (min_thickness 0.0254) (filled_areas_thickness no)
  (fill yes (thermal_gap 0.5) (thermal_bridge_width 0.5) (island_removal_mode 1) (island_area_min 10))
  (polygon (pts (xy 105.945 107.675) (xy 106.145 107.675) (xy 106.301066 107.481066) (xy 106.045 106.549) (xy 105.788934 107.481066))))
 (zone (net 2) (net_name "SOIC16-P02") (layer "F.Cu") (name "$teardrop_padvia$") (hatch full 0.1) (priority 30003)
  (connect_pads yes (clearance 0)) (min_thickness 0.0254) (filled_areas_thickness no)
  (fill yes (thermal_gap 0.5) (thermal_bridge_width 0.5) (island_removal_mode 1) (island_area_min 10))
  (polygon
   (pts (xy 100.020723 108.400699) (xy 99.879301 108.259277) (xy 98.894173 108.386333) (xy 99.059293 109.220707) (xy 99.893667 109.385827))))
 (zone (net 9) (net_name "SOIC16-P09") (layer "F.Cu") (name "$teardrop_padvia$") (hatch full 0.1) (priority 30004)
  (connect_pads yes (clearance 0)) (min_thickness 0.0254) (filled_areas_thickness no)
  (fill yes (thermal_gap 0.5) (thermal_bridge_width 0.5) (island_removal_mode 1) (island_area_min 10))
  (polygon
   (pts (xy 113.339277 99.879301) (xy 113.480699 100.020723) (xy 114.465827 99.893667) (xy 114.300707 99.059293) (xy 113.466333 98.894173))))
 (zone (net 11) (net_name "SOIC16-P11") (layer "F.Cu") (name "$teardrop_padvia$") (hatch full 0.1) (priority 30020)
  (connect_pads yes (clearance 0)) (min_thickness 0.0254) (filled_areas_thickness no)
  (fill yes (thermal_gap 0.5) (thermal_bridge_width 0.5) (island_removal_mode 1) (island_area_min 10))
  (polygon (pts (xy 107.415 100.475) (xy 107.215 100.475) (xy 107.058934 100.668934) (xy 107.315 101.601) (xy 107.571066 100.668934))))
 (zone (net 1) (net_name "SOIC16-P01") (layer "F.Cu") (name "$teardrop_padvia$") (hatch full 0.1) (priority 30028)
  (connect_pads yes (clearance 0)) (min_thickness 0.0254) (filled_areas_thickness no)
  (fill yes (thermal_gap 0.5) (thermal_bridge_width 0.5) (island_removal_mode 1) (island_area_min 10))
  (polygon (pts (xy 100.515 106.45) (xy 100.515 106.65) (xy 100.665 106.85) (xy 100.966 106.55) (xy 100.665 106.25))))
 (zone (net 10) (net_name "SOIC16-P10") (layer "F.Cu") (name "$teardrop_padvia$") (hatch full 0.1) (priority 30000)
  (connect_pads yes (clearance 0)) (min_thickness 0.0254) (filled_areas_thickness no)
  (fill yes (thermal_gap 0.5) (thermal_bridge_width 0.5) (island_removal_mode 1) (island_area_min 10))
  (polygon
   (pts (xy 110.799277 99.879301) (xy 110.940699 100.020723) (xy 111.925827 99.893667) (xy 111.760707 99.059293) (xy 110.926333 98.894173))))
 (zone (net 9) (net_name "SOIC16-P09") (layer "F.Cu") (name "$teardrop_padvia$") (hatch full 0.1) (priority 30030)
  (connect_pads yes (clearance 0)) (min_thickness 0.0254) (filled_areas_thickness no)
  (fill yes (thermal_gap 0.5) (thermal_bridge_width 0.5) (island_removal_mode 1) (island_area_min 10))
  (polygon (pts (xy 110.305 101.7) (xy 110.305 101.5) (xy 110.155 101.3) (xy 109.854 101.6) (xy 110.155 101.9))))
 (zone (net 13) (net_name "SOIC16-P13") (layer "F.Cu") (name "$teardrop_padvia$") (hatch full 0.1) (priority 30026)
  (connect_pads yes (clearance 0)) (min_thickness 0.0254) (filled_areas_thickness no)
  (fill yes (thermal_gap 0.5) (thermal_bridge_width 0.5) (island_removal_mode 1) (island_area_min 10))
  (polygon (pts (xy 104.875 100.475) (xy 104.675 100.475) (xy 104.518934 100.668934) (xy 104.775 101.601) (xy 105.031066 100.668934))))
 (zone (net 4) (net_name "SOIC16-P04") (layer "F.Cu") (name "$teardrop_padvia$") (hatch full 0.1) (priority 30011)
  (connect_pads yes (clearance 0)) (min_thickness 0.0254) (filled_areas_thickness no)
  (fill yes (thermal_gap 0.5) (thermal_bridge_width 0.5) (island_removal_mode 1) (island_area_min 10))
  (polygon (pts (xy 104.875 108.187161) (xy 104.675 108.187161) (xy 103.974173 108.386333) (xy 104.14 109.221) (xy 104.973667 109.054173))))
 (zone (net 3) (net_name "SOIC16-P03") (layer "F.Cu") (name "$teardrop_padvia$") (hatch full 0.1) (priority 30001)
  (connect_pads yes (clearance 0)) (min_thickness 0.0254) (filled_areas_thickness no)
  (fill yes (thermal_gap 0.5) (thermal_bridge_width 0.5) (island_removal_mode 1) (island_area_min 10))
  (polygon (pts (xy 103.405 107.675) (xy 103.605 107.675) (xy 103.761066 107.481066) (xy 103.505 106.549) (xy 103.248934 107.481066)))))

